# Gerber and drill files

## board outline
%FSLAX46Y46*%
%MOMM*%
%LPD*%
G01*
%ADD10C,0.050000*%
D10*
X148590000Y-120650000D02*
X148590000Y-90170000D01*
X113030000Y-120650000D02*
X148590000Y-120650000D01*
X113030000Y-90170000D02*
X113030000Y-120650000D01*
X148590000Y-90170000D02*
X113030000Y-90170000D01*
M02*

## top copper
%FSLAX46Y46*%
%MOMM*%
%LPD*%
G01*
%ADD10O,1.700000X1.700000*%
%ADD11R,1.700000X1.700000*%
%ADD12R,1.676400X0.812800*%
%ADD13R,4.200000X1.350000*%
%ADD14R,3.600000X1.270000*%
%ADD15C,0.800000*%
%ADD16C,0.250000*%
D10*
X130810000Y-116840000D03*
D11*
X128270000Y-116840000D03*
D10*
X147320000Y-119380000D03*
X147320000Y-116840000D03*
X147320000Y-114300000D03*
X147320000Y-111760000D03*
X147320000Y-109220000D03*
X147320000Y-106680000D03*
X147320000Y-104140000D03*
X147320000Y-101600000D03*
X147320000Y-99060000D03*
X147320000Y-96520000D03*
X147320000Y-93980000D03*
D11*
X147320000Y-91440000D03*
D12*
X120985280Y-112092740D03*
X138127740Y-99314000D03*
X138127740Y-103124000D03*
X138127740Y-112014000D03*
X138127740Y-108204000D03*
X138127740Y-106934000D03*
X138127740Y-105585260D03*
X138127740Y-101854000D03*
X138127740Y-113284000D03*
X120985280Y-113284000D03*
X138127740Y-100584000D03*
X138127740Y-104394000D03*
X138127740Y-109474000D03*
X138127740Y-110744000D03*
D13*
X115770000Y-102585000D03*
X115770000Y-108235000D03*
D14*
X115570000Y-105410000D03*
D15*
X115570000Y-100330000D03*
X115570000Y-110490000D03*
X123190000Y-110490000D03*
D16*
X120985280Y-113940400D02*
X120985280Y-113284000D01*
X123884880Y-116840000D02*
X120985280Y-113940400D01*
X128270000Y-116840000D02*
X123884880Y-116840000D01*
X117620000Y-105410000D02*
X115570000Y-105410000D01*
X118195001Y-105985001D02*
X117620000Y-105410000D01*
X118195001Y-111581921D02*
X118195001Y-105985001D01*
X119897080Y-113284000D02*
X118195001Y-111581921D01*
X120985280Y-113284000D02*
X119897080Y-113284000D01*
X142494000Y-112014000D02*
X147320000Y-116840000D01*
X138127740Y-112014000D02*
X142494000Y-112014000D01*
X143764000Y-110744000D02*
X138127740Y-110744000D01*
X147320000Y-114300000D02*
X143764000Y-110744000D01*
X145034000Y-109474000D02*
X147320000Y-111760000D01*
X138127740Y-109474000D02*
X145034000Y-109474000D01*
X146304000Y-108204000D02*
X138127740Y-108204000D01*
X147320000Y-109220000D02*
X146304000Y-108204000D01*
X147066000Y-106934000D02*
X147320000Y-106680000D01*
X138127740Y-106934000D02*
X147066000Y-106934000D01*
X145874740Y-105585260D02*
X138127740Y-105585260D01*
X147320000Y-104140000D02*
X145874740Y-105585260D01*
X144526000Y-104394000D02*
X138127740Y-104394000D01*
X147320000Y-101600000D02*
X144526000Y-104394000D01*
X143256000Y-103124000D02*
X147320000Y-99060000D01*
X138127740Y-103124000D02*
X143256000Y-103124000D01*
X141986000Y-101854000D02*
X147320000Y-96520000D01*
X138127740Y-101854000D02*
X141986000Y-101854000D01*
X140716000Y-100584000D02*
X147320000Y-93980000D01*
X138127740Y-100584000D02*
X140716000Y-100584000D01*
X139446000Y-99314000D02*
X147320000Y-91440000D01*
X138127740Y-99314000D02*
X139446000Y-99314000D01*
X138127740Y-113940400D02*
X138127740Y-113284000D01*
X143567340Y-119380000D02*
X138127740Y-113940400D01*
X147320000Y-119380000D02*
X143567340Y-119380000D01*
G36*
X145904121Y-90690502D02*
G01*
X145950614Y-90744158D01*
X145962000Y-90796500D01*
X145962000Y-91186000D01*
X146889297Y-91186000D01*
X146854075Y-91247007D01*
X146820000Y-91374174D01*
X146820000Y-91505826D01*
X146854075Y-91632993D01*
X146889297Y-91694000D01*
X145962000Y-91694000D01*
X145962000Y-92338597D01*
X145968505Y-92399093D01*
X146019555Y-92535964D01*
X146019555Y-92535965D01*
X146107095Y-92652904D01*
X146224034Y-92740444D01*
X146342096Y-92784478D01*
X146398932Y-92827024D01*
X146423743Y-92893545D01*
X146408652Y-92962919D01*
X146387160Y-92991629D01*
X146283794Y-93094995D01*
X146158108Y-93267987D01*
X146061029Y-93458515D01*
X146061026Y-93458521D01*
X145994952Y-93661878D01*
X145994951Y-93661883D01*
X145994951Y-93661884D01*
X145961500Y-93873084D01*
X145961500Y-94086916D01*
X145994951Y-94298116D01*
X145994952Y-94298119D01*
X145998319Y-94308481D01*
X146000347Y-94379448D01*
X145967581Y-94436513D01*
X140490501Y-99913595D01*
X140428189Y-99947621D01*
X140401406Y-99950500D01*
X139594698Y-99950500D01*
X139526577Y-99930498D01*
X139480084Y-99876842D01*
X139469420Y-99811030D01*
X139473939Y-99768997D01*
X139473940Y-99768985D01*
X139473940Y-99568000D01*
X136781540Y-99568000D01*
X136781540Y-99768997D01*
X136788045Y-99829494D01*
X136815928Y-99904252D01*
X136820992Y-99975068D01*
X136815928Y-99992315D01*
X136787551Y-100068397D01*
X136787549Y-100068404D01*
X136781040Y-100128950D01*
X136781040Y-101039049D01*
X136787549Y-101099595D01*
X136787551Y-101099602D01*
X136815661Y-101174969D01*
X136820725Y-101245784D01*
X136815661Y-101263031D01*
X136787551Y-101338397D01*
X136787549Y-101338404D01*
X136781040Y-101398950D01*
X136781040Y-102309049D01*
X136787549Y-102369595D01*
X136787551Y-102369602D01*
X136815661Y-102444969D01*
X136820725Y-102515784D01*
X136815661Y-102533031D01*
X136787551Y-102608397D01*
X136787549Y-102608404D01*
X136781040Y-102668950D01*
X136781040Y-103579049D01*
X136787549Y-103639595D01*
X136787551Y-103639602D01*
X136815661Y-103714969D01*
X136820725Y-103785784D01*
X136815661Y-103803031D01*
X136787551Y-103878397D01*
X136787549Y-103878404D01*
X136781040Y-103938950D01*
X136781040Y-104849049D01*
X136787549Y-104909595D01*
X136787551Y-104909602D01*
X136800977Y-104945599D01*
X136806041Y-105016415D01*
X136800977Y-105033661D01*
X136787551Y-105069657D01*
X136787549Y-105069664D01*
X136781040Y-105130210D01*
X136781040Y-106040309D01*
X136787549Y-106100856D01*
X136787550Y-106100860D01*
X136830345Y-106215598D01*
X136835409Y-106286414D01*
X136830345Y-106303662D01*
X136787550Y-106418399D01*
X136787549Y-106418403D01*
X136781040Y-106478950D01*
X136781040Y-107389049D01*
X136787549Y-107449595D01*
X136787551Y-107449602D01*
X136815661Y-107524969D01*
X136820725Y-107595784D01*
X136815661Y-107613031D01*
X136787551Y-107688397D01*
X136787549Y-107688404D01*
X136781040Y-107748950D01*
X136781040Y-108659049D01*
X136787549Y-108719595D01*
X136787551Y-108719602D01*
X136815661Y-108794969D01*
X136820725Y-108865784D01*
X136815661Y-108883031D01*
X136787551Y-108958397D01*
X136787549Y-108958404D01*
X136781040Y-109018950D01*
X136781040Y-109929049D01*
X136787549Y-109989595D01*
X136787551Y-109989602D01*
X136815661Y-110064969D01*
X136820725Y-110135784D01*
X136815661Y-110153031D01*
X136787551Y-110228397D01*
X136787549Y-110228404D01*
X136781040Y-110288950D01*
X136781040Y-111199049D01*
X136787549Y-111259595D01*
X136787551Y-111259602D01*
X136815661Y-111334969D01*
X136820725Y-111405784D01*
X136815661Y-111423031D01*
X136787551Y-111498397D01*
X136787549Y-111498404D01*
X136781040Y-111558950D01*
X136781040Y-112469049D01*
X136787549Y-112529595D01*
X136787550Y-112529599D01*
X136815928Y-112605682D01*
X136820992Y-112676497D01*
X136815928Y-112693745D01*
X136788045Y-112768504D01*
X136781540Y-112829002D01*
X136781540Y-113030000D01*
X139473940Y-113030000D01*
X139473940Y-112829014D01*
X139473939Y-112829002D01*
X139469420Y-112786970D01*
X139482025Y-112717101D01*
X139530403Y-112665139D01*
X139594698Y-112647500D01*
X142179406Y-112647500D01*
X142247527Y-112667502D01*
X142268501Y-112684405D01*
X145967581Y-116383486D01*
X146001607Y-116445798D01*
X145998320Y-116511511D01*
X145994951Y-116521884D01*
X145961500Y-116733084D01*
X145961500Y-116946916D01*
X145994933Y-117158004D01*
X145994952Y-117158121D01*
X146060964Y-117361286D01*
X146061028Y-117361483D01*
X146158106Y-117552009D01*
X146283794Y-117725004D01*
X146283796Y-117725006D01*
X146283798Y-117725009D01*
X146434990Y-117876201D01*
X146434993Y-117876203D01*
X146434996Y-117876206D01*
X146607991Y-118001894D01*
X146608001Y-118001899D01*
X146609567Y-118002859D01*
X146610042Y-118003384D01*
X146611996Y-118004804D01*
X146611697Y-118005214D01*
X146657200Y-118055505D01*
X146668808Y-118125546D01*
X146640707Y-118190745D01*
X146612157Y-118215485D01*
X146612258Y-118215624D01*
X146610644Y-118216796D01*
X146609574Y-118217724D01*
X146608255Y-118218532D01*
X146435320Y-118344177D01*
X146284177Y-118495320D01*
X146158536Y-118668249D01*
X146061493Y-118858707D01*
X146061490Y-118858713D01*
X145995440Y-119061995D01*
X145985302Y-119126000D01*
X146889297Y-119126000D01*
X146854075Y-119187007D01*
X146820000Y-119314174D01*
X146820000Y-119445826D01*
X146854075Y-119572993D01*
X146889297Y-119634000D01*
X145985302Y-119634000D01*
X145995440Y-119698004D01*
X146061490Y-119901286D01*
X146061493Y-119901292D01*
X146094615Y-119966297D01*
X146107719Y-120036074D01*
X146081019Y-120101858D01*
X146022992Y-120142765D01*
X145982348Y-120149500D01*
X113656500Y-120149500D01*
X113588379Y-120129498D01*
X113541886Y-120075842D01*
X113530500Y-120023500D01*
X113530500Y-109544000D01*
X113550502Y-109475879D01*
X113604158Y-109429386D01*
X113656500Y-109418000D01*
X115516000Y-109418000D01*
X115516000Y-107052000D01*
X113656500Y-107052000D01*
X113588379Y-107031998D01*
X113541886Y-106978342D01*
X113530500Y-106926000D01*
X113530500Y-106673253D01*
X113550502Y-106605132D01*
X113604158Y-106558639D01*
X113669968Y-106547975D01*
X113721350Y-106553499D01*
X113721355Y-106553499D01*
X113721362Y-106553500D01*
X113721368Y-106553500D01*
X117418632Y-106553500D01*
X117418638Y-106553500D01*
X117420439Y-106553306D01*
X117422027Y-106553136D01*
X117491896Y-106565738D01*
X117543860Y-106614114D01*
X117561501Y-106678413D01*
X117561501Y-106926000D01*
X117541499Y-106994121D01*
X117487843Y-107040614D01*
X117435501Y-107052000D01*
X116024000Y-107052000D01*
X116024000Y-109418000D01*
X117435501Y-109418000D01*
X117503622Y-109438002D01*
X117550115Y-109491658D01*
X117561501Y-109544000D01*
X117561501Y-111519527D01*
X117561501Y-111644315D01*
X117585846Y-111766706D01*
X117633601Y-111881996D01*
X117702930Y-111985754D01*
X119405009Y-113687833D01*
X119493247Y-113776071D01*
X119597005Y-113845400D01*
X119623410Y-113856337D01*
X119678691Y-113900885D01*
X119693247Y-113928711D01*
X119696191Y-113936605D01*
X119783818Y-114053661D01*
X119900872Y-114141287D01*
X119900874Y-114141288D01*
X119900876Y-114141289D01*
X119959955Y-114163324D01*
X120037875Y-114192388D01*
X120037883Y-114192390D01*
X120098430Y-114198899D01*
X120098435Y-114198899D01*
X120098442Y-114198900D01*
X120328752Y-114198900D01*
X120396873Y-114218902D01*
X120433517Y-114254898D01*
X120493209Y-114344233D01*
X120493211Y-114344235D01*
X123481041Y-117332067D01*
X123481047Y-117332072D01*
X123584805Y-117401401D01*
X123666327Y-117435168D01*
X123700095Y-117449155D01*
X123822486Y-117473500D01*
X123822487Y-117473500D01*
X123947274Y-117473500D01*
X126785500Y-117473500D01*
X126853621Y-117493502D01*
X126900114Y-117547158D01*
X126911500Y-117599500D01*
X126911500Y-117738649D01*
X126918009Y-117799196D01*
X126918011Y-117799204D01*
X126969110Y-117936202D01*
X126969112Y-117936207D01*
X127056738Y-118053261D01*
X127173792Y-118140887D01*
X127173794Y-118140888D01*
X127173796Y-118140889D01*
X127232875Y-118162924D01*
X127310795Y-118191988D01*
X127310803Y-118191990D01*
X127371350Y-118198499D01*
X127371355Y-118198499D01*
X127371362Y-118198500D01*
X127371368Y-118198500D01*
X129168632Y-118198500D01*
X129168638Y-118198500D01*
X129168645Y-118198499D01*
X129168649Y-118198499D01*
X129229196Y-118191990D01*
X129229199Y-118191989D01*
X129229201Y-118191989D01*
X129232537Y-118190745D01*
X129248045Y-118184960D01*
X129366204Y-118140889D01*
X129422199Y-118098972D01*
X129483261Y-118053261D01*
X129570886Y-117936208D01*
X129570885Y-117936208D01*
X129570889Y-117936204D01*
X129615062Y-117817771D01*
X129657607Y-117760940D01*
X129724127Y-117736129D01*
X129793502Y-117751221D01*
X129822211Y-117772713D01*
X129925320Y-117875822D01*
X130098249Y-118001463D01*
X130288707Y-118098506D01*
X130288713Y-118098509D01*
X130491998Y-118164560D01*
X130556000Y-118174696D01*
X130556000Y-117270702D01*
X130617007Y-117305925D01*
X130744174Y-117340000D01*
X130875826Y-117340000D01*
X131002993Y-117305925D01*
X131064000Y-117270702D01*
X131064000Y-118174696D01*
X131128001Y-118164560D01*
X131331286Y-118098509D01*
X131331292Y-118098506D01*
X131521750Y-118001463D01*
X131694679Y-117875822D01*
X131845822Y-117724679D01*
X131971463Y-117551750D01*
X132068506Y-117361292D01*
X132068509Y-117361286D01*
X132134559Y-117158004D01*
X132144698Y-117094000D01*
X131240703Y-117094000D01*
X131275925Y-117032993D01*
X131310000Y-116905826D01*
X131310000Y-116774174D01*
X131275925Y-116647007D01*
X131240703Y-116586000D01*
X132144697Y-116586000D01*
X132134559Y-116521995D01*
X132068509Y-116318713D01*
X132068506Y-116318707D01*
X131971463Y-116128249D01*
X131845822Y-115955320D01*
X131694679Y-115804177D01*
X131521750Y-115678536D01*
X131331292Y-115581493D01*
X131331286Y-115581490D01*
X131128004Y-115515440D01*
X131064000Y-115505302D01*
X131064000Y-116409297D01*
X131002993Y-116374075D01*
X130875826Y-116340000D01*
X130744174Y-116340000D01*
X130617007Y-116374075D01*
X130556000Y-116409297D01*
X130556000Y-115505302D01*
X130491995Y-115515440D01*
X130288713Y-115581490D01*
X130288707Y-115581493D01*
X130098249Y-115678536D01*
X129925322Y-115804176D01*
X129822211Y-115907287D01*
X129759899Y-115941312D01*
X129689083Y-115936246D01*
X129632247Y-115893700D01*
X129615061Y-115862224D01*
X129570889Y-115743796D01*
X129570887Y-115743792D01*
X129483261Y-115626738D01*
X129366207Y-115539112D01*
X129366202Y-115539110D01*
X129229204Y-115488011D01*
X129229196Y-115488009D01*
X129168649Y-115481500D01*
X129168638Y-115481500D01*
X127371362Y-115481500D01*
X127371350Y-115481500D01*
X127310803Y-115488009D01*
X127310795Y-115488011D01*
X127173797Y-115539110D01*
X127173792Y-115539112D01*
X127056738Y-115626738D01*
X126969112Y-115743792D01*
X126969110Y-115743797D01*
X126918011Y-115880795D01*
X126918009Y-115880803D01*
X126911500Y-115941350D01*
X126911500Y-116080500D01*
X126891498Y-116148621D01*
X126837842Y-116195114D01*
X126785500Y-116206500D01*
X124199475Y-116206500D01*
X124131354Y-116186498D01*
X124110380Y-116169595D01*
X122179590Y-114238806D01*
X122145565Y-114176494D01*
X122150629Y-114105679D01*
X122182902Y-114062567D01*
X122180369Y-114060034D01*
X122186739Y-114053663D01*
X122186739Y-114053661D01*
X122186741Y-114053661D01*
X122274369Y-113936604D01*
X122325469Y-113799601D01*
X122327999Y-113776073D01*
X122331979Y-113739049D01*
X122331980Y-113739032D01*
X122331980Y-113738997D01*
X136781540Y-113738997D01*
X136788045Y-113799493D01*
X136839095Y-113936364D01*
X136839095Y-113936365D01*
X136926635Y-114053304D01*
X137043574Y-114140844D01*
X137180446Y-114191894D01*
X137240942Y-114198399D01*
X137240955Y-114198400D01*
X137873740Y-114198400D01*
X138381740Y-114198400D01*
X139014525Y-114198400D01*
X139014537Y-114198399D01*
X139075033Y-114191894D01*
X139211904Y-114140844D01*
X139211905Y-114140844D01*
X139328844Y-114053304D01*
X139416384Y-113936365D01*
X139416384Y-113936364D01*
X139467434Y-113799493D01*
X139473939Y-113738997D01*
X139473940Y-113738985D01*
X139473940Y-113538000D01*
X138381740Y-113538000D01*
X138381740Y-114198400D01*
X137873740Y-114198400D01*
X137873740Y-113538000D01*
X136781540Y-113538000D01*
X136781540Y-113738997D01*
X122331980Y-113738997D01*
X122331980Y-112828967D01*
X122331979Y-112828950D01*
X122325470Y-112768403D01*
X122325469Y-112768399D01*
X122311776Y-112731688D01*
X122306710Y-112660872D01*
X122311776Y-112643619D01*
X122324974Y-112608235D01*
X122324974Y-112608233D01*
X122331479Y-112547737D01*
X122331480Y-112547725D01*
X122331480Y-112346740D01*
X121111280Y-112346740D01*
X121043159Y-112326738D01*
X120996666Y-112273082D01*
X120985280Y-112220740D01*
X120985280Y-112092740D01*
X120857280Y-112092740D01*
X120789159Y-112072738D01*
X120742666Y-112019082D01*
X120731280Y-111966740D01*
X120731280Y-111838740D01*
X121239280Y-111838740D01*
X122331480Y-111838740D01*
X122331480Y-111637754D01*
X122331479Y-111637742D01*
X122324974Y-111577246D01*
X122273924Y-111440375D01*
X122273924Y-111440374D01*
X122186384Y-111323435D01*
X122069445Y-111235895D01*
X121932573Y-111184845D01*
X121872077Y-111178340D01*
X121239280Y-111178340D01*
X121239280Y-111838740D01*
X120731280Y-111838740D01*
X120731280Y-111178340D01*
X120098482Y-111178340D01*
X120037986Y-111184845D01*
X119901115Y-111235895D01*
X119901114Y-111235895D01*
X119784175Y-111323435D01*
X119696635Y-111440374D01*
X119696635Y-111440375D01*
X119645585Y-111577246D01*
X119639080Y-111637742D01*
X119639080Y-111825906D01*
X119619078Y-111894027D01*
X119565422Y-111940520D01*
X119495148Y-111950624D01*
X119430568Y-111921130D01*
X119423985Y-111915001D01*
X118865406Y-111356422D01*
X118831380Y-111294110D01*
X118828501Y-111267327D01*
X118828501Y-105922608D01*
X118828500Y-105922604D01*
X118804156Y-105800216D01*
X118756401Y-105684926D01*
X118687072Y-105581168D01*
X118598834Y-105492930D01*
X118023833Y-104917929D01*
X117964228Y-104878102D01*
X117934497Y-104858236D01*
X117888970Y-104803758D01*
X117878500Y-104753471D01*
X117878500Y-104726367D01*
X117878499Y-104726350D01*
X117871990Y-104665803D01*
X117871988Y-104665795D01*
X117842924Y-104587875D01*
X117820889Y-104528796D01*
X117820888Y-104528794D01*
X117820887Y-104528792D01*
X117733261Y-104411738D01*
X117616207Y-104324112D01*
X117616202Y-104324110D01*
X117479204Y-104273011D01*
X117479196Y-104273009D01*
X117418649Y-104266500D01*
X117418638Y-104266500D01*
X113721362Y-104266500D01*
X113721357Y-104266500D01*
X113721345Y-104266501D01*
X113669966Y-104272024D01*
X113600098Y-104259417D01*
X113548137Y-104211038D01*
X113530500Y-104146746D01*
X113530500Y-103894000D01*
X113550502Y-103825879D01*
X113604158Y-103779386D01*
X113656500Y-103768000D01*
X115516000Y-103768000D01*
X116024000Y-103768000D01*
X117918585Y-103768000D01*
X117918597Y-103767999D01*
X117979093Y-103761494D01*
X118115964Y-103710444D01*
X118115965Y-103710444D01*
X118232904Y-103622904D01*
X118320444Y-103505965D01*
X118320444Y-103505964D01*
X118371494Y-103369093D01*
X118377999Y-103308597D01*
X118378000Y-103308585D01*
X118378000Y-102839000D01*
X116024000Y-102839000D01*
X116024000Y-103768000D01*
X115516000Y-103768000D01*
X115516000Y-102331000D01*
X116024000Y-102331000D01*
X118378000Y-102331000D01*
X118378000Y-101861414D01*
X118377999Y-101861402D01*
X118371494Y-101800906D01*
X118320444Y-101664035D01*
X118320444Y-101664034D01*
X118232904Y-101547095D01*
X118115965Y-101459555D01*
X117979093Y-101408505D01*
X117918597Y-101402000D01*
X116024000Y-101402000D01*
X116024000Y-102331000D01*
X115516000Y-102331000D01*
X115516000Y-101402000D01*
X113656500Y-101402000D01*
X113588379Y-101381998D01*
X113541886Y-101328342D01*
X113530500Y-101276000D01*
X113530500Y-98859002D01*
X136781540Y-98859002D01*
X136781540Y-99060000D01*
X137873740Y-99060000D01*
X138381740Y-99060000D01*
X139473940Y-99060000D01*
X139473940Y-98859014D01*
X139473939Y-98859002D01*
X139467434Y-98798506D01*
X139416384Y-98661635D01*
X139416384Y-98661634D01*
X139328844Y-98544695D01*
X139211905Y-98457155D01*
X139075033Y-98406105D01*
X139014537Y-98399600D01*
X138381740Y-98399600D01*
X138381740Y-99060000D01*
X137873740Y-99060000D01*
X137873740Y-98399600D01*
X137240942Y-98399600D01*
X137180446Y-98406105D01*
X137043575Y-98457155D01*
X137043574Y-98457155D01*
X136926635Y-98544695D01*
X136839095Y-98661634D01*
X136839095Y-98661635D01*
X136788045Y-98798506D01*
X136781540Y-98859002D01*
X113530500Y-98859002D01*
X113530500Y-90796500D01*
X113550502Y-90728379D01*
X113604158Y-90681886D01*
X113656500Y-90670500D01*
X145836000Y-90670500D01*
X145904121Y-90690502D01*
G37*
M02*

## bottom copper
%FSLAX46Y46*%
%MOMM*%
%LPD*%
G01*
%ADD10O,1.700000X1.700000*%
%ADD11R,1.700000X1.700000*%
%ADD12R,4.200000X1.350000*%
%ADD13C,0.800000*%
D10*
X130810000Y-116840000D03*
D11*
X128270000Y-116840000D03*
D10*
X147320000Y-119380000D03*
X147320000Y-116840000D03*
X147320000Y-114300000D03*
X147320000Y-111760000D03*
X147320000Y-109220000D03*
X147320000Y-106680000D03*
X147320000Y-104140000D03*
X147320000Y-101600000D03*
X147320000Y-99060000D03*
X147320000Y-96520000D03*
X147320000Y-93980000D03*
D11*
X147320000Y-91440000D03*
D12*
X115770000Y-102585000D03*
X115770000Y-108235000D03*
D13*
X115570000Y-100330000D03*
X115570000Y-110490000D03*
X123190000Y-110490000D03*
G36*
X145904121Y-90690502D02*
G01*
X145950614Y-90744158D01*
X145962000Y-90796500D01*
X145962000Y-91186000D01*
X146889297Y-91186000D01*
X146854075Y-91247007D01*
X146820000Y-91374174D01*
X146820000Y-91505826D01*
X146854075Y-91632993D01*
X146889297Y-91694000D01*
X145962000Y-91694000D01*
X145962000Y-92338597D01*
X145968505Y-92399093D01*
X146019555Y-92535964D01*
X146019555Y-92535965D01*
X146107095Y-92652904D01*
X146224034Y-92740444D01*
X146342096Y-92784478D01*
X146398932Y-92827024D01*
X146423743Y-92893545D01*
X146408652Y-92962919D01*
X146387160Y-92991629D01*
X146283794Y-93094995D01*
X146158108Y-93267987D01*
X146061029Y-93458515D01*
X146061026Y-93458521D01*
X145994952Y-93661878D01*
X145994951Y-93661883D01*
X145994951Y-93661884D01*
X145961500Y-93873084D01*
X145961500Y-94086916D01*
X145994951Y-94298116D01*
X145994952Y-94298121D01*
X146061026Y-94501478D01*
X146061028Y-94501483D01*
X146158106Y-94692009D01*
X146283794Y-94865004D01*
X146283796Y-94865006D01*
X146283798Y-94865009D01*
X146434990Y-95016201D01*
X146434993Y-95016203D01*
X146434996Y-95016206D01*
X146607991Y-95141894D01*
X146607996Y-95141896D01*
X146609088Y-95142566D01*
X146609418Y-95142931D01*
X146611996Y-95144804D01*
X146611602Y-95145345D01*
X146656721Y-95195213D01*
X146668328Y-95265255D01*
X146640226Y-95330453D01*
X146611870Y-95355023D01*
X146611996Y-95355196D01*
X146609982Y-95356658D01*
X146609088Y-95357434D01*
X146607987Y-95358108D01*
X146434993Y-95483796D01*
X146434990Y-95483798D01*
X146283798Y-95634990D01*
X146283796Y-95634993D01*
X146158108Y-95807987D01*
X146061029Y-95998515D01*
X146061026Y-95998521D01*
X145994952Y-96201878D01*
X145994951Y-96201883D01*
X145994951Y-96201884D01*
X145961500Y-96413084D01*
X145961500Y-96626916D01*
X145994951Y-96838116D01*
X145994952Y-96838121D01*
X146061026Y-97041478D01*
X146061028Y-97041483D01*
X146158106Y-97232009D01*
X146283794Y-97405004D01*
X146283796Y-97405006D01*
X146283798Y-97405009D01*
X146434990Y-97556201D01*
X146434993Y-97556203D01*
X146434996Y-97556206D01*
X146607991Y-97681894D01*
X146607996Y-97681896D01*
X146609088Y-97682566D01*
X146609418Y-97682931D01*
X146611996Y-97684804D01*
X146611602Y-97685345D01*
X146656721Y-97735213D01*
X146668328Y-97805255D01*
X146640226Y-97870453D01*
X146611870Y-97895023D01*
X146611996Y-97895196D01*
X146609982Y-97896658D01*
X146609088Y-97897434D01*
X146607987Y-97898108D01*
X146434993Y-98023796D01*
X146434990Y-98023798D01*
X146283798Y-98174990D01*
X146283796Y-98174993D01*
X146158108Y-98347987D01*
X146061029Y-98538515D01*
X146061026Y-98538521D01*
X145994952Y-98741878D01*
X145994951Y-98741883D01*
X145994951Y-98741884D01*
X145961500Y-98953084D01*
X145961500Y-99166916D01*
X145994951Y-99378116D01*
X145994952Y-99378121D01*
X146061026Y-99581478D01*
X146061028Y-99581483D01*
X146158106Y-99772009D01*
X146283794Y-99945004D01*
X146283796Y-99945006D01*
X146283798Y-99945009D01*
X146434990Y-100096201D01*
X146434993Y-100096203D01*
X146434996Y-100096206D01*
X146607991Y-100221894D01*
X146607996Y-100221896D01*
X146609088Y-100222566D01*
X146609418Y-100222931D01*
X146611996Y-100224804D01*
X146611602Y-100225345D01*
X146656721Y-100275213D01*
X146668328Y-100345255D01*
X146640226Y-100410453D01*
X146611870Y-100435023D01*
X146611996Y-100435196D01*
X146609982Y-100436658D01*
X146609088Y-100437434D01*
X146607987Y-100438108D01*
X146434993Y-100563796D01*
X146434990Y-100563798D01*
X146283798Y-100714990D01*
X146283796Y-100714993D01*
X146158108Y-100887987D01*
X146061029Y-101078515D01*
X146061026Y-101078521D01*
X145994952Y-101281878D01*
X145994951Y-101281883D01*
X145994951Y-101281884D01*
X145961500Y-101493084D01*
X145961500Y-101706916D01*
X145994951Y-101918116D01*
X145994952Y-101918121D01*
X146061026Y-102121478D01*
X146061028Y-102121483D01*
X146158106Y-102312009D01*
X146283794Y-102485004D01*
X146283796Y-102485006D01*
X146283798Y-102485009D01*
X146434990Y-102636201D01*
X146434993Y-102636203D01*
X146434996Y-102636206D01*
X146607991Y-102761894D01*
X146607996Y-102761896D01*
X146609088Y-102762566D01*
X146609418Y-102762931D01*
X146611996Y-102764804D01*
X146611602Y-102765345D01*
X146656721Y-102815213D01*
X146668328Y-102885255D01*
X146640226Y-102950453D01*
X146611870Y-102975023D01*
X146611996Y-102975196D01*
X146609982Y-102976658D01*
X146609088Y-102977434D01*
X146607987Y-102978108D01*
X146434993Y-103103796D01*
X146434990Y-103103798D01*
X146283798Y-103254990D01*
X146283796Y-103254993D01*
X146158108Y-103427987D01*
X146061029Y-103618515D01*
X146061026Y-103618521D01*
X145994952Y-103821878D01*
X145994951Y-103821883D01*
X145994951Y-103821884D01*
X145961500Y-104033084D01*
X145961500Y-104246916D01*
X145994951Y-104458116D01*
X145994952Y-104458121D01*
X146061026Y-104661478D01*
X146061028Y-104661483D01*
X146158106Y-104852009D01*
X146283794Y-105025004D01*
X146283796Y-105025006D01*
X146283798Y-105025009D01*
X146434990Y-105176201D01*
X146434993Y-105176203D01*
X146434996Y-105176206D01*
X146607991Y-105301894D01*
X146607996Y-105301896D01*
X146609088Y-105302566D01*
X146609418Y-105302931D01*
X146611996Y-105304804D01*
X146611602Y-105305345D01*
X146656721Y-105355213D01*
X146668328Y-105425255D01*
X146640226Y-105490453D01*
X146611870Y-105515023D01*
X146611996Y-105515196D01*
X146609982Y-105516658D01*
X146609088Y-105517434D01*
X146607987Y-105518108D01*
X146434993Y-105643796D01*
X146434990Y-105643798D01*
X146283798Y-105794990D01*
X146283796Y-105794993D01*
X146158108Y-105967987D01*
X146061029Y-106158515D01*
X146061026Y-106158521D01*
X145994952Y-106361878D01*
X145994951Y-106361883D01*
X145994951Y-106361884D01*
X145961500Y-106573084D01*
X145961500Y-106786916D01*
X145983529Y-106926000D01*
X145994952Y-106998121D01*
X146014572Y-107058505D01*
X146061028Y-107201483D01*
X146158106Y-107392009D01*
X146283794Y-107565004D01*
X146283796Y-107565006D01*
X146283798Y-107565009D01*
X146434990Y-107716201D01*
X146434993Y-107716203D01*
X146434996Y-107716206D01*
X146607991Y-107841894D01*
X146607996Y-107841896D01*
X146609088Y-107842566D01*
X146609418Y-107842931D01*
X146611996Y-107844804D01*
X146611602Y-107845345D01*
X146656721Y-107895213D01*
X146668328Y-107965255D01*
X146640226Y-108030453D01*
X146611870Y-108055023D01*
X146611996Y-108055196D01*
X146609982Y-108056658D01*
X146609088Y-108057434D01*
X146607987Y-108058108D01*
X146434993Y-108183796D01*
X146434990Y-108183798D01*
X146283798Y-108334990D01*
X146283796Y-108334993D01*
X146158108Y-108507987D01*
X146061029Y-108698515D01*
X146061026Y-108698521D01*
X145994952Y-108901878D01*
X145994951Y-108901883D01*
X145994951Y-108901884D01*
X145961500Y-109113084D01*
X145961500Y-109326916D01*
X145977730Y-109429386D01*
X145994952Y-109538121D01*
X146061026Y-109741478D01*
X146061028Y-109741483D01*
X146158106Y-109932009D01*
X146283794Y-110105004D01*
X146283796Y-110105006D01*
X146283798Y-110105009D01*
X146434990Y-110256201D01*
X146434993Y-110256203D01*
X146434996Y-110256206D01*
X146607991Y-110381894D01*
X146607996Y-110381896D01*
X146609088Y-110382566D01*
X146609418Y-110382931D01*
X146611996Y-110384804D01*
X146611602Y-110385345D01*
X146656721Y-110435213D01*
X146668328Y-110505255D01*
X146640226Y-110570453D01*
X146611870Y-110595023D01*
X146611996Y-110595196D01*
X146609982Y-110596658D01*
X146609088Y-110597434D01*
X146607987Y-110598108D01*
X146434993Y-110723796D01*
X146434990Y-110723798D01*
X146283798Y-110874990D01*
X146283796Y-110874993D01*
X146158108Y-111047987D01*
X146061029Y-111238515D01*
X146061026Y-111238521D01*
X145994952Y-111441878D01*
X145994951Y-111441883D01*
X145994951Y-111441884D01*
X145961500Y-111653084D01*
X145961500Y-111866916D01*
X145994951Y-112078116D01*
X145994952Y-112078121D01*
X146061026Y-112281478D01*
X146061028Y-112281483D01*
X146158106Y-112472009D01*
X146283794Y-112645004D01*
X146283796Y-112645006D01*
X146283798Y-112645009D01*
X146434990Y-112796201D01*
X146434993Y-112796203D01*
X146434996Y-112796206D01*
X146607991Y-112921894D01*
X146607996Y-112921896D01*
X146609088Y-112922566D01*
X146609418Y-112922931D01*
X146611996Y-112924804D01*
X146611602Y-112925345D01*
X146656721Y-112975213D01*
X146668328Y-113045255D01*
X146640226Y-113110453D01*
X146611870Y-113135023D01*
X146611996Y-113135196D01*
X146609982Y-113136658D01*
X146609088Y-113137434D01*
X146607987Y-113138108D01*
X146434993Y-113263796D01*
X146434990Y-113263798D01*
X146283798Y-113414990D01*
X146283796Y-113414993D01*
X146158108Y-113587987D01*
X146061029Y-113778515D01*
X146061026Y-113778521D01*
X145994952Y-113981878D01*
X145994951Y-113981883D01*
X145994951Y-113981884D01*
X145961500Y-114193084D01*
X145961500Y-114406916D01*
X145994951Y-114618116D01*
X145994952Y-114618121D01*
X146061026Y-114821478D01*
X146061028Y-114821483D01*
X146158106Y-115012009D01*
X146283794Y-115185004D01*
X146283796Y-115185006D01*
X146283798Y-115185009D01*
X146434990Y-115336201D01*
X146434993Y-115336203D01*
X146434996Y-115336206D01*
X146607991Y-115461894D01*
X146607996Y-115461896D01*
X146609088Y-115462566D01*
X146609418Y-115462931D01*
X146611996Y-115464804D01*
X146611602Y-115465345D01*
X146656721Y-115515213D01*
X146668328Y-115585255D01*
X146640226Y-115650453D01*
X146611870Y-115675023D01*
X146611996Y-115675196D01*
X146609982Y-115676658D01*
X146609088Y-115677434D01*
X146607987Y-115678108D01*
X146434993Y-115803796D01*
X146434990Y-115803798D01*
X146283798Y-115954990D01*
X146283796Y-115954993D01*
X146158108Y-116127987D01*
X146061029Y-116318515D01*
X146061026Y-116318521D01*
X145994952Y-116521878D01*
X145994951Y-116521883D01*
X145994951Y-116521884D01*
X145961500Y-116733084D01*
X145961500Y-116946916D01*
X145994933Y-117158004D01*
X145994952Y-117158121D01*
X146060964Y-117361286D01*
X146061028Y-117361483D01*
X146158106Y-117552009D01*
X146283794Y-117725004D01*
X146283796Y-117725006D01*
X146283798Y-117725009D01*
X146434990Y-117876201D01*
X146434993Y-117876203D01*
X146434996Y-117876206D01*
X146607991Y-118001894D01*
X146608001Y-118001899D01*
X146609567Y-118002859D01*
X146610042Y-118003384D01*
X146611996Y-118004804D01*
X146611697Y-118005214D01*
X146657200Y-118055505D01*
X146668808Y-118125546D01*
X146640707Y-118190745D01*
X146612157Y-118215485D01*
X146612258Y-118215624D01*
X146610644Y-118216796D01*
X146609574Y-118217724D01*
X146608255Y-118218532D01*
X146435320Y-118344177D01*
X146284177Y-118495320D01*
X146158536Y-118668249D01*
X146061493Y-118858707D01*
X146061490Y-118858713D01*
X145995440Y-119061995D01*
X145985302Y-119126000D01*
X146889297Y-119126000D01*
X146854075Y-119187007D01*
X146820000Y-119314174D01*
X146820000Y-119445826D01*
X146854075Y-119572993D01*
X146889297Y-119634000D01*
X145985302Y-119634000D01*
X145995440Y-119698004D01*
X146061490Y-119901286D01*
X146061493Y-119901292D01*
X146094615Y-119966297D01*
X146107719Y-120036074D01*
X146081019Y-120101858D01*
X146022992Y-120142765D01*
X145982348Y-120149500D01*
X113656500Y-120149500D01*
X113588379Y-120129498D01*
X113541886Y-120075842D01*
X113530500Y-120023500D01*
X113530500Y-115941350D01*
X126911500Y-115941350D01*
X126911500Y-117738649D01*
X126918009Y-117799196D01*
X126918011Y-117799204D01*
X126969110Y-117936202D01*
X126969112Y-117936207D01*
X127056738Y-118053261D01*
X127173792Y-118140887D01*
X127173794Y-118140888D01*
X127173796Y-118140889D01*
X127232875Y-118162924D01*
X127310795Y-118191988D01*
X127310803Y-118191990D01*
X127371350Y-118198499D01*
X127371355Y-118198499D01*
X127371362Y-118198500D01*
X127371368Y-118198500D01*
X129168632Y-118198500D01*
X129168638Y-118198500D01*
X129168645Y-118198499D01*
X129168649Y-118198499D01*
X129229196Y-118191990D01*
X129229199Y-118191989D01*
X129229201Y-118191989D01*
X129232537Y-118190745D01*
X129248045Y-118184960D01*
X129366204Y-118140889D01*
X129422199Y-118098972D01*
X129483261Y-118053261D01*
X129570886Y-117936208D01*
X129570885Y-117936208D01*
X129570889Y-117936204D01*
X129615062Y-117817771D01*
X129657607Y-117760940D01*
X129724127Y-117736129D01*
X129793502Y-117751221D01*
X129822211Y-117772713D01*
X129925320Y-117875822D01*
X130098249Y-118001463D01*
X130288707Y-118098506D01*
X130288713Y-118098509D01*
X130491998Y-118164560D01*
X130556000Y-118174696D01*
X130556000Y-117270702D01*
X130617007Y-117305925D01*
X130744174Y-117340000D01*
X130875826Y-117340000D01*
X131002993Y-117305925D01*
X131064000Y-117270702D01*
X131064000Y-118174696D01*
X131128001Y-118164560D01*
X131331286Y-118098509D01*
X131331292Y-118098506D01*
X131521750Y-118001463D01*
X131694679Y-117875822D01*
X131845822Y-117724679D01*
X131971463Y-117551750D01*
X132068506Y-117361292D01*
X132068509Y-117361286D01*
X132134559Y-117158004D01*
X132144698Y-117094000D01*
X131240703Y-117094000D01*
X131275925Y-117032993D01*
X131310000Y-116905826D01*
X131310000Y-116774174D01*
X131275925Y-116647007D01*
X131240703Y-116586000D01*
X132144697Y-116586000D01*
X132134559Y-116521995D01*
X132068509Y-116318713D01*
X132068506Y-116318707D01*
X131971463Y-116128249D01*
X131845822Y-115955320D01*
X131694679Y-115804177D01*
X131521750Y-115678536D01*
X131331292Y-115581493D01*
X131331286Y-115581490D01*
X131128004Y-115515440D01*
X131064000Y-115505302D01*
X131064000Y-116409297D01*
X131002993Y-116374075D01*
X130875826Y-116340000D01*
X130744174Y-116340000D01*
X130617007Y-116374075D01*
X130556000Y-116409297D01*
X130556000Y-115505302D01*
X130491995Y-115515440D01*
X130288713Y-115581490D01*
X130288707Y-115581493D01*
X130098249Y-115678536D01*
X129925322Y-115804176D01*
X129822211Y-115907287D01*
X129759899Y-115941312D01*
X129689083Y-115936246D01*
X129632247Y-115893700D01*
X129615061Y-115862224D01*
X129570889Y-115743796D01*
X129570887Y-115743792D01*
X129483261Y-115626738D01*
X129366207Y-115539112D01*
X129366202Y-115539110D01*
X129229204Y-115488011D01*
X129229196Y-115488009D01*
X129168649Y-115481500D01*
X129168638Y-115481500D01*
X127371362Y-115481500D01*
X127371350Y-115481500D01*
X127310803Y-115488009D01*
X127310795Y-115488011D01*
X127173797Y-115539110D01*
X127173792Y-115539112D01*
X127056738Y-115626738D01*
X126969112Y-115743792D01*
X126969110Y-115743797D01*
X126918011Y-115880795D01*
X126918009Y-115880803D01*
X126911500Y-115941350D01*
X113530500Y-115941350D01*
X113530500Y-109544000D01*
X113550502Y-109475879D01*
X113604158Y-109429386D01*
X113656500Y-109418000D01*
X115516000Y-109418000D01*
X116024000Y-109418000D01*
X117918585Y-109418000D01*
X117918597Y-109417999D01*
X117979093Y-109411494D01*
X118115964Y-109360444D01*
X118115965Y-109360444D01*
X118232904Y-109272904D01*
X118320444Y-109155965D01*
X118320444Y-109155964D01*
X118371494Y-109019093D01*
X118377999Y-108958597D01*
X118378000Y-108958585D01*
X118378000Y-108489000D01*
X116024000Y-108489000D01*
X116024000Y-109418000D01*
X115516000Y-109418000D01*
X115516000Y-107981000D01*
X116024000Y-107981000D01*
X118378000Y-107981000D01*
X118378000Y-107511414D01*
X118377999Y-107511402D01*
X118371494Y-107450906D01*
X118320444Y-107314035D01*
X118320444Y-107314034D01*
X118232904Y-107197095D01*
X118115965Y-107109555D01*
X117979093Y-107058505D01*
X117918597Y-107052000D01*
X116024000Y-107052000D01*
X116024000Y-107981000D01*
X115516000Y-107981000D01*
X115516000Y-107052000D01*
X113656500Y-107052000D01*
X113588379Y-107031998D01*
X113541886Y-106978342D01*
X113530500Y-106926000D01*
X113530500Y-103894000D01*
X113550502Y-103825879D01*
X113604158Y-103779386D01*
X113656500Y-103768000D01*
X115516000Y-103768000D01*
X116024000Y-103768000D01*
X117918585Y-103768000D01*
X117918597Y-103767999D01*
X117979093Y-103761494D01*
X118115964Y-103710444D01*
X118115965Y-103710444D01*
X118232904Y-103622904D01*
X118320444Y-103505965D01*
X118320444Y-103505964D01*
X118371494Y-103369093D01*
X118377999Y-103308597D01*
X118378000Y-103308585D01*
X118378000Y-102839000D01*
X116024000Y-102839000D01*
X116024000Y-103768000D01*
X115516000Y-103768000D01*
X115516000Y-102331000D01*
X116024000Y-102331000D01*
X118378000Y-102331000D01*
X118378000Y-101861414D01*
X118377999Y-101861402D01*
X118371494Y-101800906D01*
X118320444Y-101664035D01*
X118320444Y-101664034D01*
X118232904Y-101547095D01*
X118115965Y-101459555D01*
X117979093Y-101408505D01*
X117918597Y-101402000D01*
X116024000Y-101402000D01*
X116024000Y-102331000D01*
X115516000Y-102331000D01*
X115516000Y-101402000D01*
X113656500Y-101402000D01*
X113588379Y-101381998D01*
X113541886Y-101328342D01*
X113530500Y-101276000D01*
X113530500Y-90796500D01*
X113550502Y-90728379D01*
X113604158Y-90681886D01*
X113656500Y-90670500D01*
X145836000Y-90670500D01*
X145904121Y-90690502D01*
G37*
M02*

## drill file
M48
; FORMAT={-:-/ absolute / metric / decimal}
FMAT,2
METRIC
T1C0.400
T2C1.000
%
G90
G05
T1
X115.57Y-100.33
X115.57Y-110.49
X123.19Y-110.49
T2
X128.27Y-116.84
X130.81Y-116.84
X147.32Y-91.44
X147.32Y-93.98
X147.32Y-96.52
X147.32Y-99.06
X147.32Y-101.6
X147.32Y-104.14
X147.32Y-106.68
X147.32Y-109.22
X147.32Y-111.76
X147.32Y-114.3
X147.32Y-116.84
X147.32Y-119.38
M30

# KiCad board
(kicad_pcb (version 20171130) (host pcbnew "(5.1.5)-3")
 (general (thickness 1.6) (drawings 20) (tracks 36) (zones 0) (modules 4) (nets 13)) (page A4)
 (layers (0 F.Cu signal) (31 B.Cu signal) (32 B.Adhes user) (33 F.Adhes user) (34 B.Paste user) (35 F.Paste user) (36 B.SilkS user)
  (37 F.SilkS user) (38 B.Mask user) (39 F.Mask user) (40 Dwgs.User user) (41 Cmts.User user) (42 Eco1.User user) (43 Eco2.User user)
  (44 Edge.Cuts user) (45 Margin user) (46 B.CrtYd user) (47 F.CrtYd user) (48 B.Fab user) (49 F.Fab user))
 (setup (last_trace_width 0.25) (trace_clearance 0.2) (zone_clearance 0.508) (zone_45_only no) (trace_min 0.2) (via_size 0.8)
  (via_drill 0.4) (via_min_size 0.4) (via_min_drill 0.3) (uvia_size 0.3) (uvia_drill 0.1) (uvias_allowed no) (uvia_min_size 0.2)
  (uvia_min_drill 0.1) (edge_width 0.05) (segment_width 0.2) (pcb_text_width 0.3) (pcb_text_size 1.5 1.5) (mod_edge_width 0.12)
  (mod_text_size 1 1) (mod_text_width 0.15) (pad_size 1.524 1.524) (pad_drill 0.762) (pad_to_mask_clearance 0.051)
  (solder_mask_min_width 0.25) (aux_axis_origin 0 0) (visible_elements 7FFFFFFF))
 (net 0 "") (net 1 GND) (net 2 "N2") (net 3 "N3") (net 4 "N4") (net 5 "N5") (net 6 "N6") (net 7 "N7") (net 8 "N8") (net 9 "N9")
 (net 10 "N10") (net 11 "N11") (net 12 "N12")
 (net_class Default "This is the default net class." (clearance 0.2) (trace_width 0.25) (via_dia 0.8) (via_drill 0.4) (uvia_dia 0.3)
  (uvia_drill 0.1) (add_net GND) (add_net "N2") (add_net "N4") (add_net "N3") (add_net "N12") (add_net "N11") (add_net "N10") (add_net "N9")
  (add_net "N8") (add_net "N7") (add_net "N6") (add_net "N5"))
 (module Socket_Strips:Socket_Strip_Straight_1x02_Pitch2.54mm (layer F.Cu) (at 128.27 116.84 90)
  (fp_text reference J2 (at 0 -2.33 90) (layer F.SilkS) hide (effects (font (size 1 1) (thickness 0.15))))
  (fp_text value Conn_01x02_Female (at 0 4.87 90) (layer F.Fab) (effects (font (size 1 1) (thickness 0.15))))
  (pad 2 thru_hole oval (at 0 2.54 90) (size 1.7 1.7) (drill 1) (layers *.Cu *.Mask) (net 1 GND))
  (pad 1 thru_hole rect (at 0 0 90) (size 1.7 1.7) (drill 1) (layers *.Cu *.Mask) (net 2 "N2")))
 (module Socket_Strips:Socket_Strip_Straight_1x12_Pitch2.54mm (layer F.Cu) (at 147.32 91.44)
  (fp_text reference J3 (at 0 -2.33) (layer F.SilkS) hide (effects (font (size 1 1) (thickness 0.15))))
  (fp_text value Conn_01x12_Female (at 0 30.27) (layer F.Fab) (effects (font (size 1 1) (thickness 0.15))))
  (pad 12 thru_hole oval (at 0 27.94) (size 1.7 1.7) (drill 1) (layers *.Cu *.Mask) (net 1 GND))
  (pad 11 thru_hole oval (at 0 25.4) (size 1.7 1.7) (drill 1) (layers *.Cu *.Mask) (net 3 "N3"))
  (pad 10 thru_hole oval (at 0 22.86) (size 1.7 1.7) (drill 1) (layers *.Cu *.Mask) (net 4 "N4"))
  (pad 9 thru_hole oval (at 0 20.32) (size 1.7 1.7) (drill 1) (layers *.Cu *.Mask) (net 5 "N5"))
  (pad 8 thru_hole oval (at 0 17.78) (size 1.7 1.7) (drill 1) (layers *.Cu *.Mask) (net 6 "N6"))
  (pad 7 thru_hole oval (at 0 15.24) (size 1.7 1.7) (drill 1) (layers *.Cu *.Mask) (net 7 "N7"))
  (pad 6 thru_hole oval (at 0 12.7) (size 1.7 1.7) (drill 1) (layers *.Cu *.Mask) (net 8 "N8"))
  (pad 5 thru_hole oval (at 0 10.16) (size 1.7 1.7) (drill 1) (layers *.Cu *.Mask) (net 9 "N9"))
  (pad 4 thru_hole oval (at 0 7.62) (size 1.7 1.7) (drill 1) (layers *.Cu *.Mask) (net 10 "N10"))
  (pad 3 thru_hole oval (at 0 5.08) (size 1.7 1.7) (drill 1) (layers *.Cu *.Mask) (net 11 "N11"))
  (pad 2 thru_hole oval (at 0 2.54) (size 1.7 1.7) (drill 1) (layers *.Cu *.Mask) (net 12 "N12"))
  (pad 1 thru_hole rect (at 0 0) (size 1.7 1.7) (drill 1) (layers *.Cu *.Mask) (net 1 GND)))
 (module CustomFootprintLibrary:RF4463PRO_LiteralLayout (layer F.Cu) (at 129.54 106.68 180)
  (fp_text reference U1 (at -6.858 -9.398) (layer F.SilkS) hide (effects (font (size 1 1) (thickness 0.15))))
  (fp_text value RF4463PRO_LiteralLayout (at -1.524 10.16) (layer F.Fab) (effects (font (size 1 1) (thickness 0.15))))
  (pad 13 smd rect (at 8.55472 -5.41274 180) (size 1.6764 0.8128) (layers F.Cu F.Paste F.Mask) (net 1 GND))
  (pad 12 smd rect (at -8.58774 7.366 180) (size 1.6764 0.8128) (layers F.Cu F.Paste F.Mask) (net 1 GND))
  (pad 9 smd rect (at -8.58774 3.556 180) (size 1.6764 0.8128) (layers F.Cu F.Paste F.Mask) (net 10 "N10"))
  (pad 2 smd rect (at -8.58774 -5.334 180) (size 1.6764 0.8128) (layers F.Cu F.Paste F.Mask) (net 3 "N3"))
  (pad 5 smd rect (at -8.58774 -1.524 180) (size 1.6764 0.8128) (layers F.Cu F.Paste F.Mask) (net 6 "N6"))
  (pad 6 smd rect (at -8.58774 -0.254 180) (size 1.6764 0.8128) (layers F.Cu F.Paste F.Mask) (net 7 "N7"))
  (pad 7 smd rect (at -8.58774 1.09474 180) (size 1.6764 0.8128) (layers F.Cu F.Paste F.Mask) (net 8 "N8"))
  (pad 10 smd rect (at -8.58774 4.826 180) (size 1.6764 0.8128) (layers F.Cu F.Paste F.Mask) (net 11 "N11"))
  (pad 1 smd rect (at -8.58774 -6.604 180) (size 1.6764 0.8128) (layers F.Cu F.Paste F.Mask) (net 1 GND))
  (pad 14 smd rect (at 8.55472 -6.604 180) (size 1.6764 0.8128) (layers F.Cu F.Paste F.Mask) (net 2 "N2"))
  (pad 11 smd rect (at -8.58774 6.096 180) (size 1.6764 0.8128) (layers F.Cu F.Paste F.Mask) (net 12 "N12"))
  (pad 8 smd rect (at -8.58774 2.286 180) (size 1.6764 0.8128) (layers F.Cu F.Paste F.Mask) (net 9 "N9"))
  (pad 4 smd rect (at -8.58774 -2.794 180) (size 1.6764 0.8128) (layers F.Cu F.Paste F.Mask) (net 5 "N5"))
  (pad 3 smd rect (at -8.58774 -4.064 180) (size 1.6764 0.8128) (layers F.Cu F.Paste F.Mask) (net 4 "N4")))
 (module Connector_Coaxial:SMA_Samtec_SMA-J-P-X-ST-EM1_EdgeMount (layer F.Cu) (at 115.77 105.41 270)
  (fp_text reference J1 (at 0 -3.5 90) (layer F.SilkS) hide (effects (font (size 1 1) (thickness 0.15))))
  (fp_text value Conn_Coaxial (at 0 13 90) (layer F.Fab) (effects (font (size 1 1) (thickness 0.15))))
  (pad 2 smd rect (at -2.825 0 270) (size 1.35 4.2) (layers B.Cu B.Paste B.Mask) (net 1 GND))
  (pad 2 smd rect (at 2.825 0 270) (size 1.35 4.2) (layers B.Cu B.Paste B.Mask) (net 1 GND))
  (pad 2 smd rect (at -2.825 0 270) (size 1.35 4.2) (layers F.Cu F.Paste F.Mask) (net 1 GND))
  (pad 2 smd rect (at 2.825 0 270) (size 1.35 4.2) (layers F.Cu F.Paste F.Mask) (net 1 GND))
  (pad 1 smd rect (at 0 0.2 270) (size 1.27 3.6) (layers F.Cu F.Paste F.Mask) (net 2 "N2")))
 (gr_line (start 148.59 120.65) (end 148.59 90.17) (layer Edge.Cuts) (width 0.05))
 (gr_line (start 113.03 120.65) (end 148.59 120.65) (layer Edge.Cuts) (width 0.05))
 (gr_line (start 113.03 90.17) (end 113.03 120.65) (layer Edge.Cuts) (width 0.05))
 (gr_line (start 148.59 90.17) (end 113.03 90.17) (layer Edge.Cuts) (width 0.05))
 (segment (start 120.98528 113.9404) (end 120.98528 113.284) (width 0.25) (layer F.Cu) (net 2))
 (segment (start 123.88488 116.84) (end 120.98528 113.9404) (width 0.25) (layer F.Cu) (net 2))
 (segment (start 128.27 116.84) (end 123.88488 116.84) (width 0.25) (layer F.Cu) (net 2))
 (segment (start 117.62 105.41) (end 115.57 105.41) (width 0.25) (layer F.Cu) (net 2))
 (segment (start 118.195001 105.985001) (end 117.62 105.41) (width 0.25) (layer F.Cu) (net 2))
 (segment (start 118.195001 111.581921) (end 118.195001 105.985001) (width 0.25) (layer F.Cu) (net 2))
 (segment (start 119.89708 113.284) (end 118.195001 111.581921) (width 0.25) (layer F.Cu) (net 2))
 (segment (start 120.98528 113.284) (end 119.89708 113.284) (width 0.25) (layer F.Cu) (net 2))
 (segment (start 142.494 112.014) (end 147.32 116.84) (width 0.25) (layer F.Cu) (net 3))
 (segment (start 138.12774 112.014) (end 142.494 112.014) (width 0.25) (layer F.Cu) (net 3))
 (segment (start 143.764 110.744) (end 138.12774 110.744) (width 0.25) (layer F.Cu) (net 4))
 (segment (start 147.32 114.3) (end 143.764 110.744) (width 0.25) (layer F.Cu) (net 4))
 (segment (start 145.034 109.474) (end 147.32 111.76) (width 0.25) (layer F.Cu) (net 5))
 (segment (start 138.12774 109.474) (end 145.034 109.474) (width 0.25) (layer F.Cu) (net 5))
 (segment (start 146.304 108.204) (end 138.12774 108.204) (width 0.25) (layer F.Cu) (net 6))
 (segment (start 147.32 109.22) (end 146.304 108.204) (width 0.25) (layer F.Cu) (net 6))
 (segment (start 147.066 106.934) (end 147.32 106.68) (width 0.25) (layer F.Cu) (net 7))
 (segment (start 138.12774 106.934) (end 147.066 106.934) (width 0.25) (layer F.Cu) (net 7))
 (segment (start 145.87474 105.58526) (end 138.12774 105.58526) (width 0.25) (layer F.Cu) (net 8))
 (segment (start 147.32 104.14) (end 145.87474 105.58526) (width 0.25) (layer F.Cu) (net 8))
 (segment (start 144.526 104.394) (end 138.12774 104.394) (width 0.25) (layer F.Cu) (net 9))
 (segment (start 147.32 101.6) (end 144.526 104.394) (width 0.25) (layer F.Cu) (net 9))
 (segment (start 143.256 103.124) (end 147.32 99.06) (width 0.25) (layer F.Cu) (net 10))
 (segment (start 138.12774 103.124) (end 143.256 103.124) (width 0.25) (layer F.Cu) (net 10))
 (segment (start 141.986 101.854) (end 147.32 96.52) (width 0.25) (layer F.Cu) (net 11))
 (segment (start 138.12774 101.854) (end 141.986 101.854) (width 0.25) (layer F.Cu) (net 11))
 (segment (start 140.716 100.584) (end 147.32 93.98) (width 0.25) (layer F.Cu) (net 12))
 (segment (start 138.12774 100.584) (end 140.716 100.584) (width 0.25) (layer F.Cu) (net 12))
 (segment (start 139.446 99.314) (end 147.32 91.44) (width 0.25) (layer F.Cu) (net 1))
 (segment (start 138.12774 99.314) (end 139.446 99.314) (width 0.25) (layer F.Cu) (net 1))
 (segment (start 138.12774 113.9404) (end 138.12774 113.284) (width 0.25) (layer F.Cu) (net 1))
 (segment (start 143.56734 119.38) (end 138.12774 113.9404) (width 0.25) (layer F.Cu) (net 1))
 (segment (start 147.32 119.38) (end 143.56734 119.38) (width 0.25) (layer F.Cu) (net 1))
 (via (at 115.57 100.33) (size 0.8) (drill 0.4) (layers F.Cu B.Cu) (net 1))
 (via (at 115.57 110.49) (size 0.8) (drill 0.4) (layers F.Cu B.Cu) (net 1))
 (via (at 123.19 110.49) (size 0.8) (drill 0.4) (layers F.Cu B.Cu) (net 1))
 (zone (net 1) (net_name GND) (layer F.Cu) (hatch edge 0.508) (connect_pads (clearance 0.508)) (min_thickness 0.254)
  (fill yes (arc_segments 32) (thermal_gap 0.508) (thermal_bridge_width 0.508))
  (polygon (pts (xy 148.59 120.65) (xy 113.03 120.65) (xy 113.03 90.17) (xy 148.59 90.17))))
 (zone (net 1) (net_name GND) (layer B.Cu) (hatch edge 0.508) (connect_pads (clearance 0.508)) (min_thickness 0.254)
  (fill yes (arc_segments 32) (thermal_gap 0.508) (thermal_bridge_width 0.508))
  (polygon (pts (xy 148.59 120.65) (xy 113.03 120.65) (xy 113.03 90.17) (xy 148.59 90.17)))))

